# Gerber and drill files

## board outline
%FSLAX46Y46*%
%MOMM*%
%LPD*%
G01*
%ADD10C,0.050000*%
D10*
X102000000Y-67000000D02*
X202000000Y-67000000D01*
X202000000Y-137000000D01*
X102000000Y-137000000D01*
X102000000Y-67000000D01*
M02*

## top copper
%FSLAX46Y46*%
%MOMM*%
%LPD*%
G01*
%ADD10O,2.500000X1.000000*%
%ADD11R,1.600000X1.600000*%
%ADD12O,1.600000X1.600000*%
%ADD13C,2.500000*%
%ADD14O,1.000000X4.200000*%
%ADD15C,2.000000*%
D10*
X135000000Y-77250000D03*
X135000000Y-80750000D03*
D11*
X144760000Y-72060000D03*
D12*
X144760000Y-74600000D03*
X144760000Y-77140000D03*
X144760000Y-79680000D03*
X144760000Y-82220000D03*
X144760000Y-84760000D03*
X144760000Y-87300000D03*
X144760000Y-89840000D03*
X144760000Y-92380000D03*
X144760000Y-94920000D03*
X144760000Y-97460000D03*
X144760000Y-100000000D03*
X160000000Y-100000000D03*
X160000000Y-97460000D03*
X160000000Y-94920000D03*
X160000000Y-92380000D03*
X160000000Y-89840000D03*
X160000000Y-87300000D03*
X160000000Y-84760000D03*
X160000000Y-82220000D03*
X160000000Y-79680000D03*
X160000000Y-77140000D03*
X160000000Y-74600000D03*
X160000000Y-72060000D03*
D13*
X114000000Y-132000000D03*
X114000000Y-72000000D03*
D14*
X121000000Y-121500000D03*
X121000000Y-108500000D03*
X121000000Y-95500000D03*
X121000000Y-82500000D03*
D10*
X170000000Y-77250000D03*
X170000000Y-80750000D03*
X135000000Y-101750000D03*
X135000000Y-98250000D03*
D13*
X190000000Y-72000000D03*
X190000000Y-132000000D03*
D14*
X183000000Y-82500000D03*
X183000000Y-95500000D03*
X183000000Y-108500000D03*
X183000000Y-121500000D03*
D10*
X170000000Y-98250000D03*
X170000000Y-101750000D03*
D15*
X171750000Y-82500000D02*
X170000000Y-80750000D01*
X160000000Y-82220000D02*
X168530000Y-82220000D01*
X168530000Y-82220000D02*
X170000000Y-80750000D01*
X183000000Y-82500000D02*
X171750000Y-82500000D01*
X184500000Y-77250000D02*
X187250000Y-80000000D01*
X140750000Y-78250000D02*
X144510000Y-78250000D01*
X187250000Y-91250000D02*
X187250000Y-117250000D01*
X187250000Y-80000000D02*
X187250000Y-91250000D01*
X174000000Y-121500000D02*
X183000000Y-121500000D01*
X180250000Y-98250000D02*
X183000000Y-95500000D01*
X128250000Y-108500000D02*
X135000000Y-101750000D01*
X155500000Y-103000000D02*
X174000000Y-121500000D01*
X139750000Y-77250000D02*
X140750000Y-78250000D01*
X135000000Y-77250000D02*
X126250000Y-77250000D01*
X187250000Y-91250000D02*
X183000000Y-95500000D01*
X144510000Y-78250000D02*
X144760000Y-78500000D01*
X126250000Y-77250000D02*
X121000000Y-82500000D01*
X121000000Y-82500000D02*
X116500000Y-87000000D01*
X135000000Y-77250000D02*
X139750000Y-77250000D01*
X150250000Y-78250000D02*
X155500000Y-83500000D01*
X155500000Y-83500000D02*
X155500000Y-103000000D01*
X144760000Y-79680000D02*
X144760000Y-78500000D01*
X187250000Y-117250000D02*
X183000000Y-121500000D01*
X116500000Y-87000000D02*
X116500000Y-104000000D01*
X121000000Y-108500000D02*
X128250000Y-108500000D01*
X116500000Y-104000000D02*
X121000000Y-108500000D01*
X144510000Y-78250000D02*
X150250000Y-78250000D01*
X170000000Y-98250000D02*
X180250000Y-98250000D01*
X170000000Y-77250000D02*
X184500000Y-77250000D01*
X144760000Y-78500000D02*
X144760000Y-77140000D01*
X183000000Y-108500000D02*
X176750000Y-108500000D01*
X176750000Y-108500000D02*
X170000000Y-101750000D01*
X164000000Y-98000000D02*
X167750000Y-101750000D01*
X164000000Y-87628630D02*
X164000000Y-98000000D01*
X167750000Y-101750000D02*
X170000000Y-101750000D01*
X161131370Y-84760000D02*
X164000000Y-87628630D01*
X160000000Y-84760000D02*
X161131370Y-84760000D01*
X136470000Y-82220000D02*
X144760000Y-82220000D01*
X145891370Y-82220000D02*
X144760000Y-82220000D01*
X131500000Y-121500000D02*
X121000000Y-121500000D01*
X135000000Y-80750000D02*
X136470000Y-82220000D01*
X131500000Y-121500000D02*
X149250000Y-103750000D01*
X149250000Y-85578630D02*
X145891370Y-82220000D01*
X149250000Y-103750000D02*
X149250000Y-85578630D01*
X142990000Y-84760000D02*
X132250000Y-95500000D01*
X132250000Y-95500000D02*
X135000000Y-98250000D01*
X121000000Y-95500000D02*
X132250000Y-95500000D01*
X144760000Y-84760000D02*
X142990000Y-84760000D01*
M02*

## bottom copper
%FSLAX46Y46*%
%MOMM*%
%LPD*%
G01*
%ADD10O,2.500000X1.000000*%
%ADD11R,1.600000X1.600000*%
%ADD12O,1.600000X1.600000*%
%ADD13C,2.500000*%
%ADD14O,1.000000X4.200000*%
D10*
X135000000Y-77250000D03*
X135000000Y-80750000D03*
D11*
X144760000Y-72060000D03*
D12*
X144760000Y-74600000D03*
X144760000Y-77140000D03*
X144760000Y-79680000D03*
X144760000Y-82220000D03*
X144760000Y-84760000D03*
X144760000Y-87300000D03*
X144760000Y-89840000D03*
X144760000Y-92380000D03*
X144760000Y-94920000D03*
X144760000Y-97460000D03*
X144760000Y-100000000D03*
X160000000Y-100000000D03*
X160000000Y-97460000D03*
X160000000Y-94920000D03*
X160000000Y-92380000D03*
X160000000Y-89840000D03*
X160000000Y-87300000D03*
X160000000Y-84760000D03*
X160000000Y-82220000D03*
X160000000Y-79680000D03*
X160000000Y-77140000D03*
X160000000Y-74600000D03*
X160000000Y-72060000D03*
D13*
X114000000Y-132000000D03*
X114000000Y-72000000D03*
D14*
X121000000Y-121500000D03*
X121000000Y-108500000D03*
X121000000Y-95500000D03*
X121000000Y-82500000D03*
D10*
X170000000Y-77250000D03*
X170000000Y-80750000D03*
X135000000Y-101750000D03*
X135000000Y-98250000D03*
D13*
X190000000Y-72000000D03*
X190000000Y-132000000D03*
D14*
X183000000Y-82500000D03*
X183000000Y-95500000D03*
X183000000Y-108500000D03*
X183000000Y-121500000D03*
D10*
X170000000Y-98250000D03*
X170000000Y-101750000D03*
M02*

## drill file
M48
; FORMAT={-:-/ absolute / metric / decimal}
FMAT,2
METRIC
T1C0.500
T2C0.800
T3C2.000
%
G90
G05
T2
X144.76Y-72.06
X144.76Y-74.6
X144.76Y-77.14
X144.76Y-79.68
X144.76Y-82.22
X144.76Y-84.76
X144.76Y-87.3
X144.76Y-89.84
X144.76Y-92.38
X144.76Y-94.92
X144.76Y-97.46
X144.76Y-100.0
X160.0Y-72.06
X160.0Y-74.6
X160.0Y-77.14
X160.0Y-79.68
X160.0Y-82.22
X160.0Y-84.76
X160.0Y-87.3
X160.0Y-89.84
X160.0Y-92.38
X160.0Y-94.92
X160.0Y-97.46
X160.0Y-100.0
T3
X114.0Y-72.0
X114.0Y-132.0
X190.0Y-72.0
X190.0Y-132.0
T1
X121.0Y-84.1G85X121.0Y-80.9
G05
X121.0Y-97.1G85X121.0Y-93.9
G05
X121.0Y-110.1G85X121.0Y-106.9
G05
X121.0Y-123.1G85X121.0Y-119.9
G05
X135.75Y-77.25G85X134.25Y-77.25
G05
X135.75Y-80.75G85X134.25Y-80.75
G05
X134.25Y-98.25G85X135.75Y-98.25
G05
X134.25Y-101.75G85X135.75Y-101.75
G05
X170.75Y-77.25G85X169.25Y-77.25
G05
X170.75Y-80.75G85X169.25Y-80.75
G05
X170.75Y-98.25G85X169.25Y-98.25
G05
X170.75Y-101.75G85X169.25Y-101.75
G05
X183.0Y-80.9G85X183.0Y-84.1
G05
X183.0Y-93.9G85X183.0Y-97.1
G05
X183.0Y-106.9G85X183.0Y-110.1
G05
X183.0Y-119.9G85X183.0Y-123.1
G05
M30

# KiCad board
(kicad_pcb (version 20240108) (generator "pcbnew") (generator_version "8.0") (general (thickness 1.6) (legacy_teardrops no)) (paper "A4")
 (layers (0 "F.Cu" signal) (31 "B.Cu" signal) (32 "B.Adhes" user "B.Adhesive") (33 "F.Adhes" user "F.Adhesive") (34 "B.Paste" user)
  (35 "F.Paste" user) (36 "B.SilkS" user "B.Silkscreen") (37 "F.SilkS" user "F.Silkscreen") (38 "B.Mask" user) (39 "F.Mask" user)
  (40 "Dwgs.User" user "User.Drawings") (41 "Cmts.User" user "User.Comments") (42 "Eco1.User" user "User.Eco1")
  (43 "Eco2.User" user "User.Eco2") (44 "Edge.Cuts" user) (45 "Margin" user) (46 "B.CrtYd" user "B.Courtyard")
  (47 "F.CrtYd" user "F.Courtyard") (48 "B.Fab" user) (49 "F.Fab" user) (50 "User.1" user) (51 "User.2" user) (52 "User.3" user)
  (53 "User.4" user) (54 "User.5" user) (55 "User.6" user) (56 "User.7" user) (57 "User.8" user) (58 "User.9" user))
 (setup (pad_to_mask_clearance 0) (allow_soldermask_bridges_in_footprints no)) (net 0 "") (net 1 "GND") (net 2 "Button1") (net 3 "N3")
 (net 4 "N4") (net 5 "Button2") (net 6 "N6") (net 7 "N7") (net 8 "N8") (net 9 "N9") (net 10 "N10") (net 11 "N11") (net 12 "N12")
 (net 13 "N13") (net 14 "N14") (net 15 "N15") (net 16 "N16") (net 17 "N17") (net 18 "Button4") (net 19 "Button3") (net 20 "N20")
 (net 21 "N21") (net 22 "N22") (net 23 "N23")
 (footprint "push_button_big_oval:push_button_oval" (layer "F.Cu") (at 135 79 90)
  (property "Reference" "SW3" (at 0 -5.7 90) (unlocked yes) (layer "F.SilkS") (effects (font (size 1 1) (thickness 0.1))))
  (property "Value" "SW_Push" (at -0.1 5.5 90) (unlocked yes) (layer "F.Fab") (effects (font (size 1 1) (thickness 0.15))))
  (pad "1" thru_hole oval (at 1.75 0 180) (size 2.5 1) (drill oval 2 0.5) (layers "*.Cu" "*.Mask") (remove_unused_layers no) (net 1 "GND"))
  (pad "2" thru_hole oval (at -1.75 0 180) (size 2.5 1) (drill oval 2 0.5) (layers "*.Cu" "*.Mask") (remove_unused_layers no)
   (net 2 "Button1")))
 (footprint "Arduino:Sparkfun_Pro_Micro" (layer "F.Cu") (at 160 100 180)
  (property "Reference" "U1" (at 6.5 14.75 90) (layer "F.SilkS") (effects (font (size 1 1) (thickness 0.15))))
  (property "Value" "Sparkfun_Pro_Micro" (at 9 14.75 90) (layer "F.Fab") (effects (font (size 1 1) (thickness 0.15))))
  (pad "1" thru_hole rect (at 15.24 27.94 180) (size 1.6 1.6) (drill 0.8) (layers "*.Cu" "*.Mask") (remove_unused_layers no) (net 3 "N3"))
  (pad "2" thru_hole oval (at 15.24 25.4 180) (size 1.6 1.6) (drill 0.8) (layers "*.Cu" "*.Mask") (remove_unused_layers no) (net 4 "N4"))
  (pad "3" thru_hole oval (at 15.24 22.86 180) (size 1.6 1.6) (drill 0.8) (layers "*.Cu" "*.Mask") (remove_unused_layers no) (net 1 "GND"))
  (pad "4" thru_hole oval (at 15.24 20.32 180) (size 1.6 1.6) (drill 0.8) (layers "*.Cu" "*.Mask") (remove_unused_layers no) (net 1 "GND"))
  (pad "5" thru_hole oval (at 15.24 17.78 180) (size 1.6 1.6) (drill 0.8) (layers "*.Cu" "*.Mask") (remove_unused_layers no)
   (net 2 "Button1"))
  (pad "6" thru_hole oval (at 15.24 15.24 180) (size 1.6 1.6) (drill 0.8) (layers "*.Cu" "*.Mask") (remove_unused_layers no)
   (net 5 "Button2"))
  (pad "7" thru_hole oval (at 15.24 12.7 180) (size 1.6 1.6) (drill 0.8) (layers "*.Cu" "*.Mask") (remove_unused_layers no) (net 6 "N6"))
  (pad "8" thru_hole oval (at 15.24 10.16 180) (size 1.6 1.6) (drill 0.8) (layers "*.Cu" "*.Mask") (remove_unused_layers no) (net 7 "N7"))
  (pad "9" thru_hole oval (at 15.24 7.62 180) (size 1.6 1.6) (drill 0.8) (layers "*.Cu" "*.Mask") (remove_unused_layers no) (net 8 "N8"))
  (pad "10" thru_hole oval (at 15.24 5.08 180) (size 1.6 1.6) (drill 0.8) (layers "*.Cu" "*.Mask") (remove_unused_layers no) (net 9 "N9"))
  (pad "11" thru_hole oval (at 15.24 2.54 180) (size 1.6 1.6) (drill 0.8) (layers "*.Cu" "*.Mask") (remove_unused_layers no) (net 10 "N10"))
  (pad "12" thru_hole oval (at 15.24 0 180) (size 1.6 1.6) (drill 0.8) (layers "*.Cu" "*.Mask") (remove_unused_layers no) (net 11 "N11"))
  (pad "13" thru_hole oval (at 0 0 180) (size 1.6 1.6) (drill 0.8) (layers "*.Cu" "*.Mask") (remove_unused_layers no) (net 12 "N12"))
  (pad "14" thru_hole oval (at 0 2.54 180) (size 1.6 1.6) (drill 0.8) (layers "*.Cu" "*.Mask") (remove_unused_layers no) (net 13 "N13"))
  (pad "15" thru_hole oval (at 0 5.08 180) (size 1.6 1.6) (drill 0.8) (layers "*.Cu" "*.Mask") (remove_unused_layers no) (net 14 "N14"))
  (pad "16" thru_hole oval (at 0 7.62 180) (size 1.6 1.6) (drill 0.8) (layers "*.Cu" "*.Mask") (remove_unused_layers no) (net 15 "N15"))
  (pad "17" thru_hole oval (at 0 10.16 180) (size 1.6 1.6) (drill 0.8) (layers "*.Cu" "*.Mask") (remove_unused_layers no) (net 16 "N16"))
  (pad "18" thru_hole oval (at 0 12.7 180) (size 1.6 1.6) (drill 0.8) (layers "*.Cu" "*.Mask") (remove_unused_layers no) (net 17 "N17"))
  (pad "19" thru_hole oval (at 0 15.24 180) (size 1.6 1.6) (drill 0.8) (layers "*.Cu" "*.Mask") (remove_unused_layers no) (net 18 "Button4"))
  (pad "20" thru_hole oval (at 0 17.78 180) (size 1.6 1.6) (drill 0.8) (layers "*.Cu" "*.Mask") (remove_unused_layers no) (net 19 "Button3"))
  (pad "21" thru_hole oval (at 0 20.32 180) (size 1.6 1.6) (drill 0.8) (layers "*.Cu" "*.Mask") (remove_unused_layers no) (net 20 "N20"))
  (pad "22" thru_hole oval (at 0 22.86 180) (size 1.6 1.6) (drill 0.8) (layers "*.Cu" "*.Mask") (remove_unused_layers no) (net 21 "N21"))
  (pad "23" thru_hole oval (at 0 25.4 180) (size 1.6 1.6) (drill 0.8) (layers "*.Cu" "*.Mask") (remove_unused_layers no) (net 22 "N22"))
  (pad "24" thru_hole oval (at 0 27.94 180) (size 1.6 1.6) (drill 0.8) (layers "*.Cu" "*.Mask") (remove_unused_layers no) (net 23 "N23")))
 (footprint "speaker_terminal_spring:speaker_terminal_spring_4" (layer "F.Cu") (at 114 102 90)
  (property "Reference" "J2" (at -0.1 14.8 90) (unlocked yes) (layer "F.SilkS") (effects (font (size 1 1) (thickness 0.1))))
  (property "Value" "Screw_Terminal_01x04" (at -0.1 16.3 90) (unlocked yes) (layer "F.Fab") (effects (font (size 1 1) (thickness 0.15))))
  (pad "" thru_hole circle (at -30 0 180) (size 2.5 2.5) (drill 2) (layers "*.Cu" "*.Mask") (remove_unused_layers no))
  (pad "" thru_hole circle (at 30 0 180) (size 2.5 2.5) (drill 2) (layers "*.Cu" "*.Mask") (remove_unused_layers no))
  (pad "1" thru_hole oval (at -19.5 7 180) (size 1 4.2) (drill oval 0.5 3.7) (layers "*.Cu" "*.Mask") (remove_unused_layers no)
   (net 2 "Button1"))
  (pad "2" thru_hole oval (at -6.5 7 180) (size 1 4.2) (drill oval 0.5 3.7) (layers "*.Cu" "*.Mask") (remove_unused_layers no) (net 1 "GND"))
  (pad "3" thru_hole oval (at 6.5 7 180) (size 1 4.2) (drill oval 0.5 3.7) (layers "*.Cu" "*.Mask") (remove_unused_layers no)
   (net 5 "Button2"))
  (pad "4" thru_hole oval (at 19.5 7 180) (size 1 4.2) (drill oval 0.5 3.7) (layers "*.Cu" "*.Mask") (remove_unused_layers no) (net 1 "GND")))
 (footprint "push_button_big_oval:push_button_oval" (layer "F.Cu") (at 170 79 90)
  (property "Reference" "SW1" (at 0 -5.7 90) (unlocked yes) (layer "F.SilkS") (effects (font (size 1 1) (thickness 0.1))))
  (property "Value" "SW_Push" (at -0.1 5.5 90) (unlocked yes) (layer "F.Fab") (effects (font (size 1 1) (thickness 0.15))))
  (pad "1" thru_hole oval (at 1.75 0 180) (size 2.5 1) (drill oval 2 0.5) (layers "*.Cu" "*.Mask") (remove_unused_layers no) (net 1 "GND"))
  (pad "2" thru_hole oval (at -1.75 0 180) (size 2.5 1) (drill oval 2 0.5) (layers "*.Cu" "*.Mask") (remove_unused_layers no)
   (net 19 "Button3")))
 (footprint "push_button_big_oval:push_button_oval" (layer "F.Cu") (at 135 100 -90)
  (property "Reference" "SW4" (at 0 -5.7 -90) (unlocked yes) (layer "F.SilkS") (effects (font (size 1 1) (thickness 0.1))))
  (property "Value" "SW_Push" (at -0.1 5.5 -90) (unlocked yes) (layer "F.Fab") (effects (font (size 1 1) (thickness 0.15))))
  (pad "1" thru_hole oval (at 1.75 0) (size 2.5 1) (drill oval 2 0.5) (layers "*.Cu" "*.Mask") (remove_unused_layers no) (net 1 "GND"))
  (pad "2" thru_hole oval (at -1.75 0) (size 2.5 1) (drill oval 2 0.5) (layers "*.Cu" "*.Mask") (remove_unused_layers no) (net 5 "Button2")))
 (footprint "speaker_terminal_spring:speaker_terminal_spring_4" (layer "F.Cu") (at 190 102 -90)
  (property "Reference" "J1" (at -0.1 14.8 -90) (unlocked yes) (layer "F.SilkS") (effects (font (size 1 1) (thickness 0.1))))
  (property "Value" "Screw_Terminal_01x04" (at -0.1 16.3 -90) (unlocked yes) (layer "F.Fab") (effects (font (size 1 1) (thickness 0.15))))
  (pad "" thru_hole circle (at -30 0) (size 2.5 2.5) (drill 2) (layers "*.Cu" "*.Mask") (remove_unused_layers no))
  (pad "" thru_hole circle (at 30 0) (size 2.5 2.5) (drill 2) (layers "*.Cu" "*.Mask") (remove_unused_layers no))
  (pad "1" thru_hole oval (at -19.5 7) (size 1 4.2) (drill oval 0.5 3.7) (layers "*.Cu" "*.Mask") (remove_unused_layers no)
   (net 19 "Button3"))
  (pad "2" thru_hole oval (at -6.5 7) (size 1 4.2) (drill oval 0.5 3.7) (layers "*.Cu" "*.Mask") (remove_unused_layers no) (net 1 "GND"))
  (pad "3" thru_hole oval (at 6.5 7) (size 1 4.2) (drill oval 0.5 3.7) (layers "*.Cu" "*.Mask") (remove_unused_layers no) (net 18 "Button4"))
  (pad "4" thru_hole oval (at 19.5 7) (size 1 4.2) (drill oval 0.5 3.7) (layers "*.Cu" "*.Mask") (remove_unused_layers no) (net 1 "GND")))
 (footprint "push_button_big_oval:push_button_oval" (layer "F.Cu") (at 170 100 90)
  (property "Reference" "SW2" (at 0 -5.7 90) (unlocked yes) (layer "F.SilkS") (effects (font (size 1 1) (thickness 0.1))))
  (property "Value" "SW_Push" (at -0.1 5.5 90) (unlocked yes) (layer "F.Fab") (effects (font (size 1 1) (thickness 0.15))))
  (pad "1" thru_hole oval (at 1.75 0 180) (size 2.5 1) (drill oval 2 0.5) (layers "*.Cu" "*.Mask") (remove_unused_layers no) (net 1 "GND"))
  (pad "2" thru_hole oval (at -1.75 0 180) (size 2.5 1) (drill oval 2 0.5) (layers "*.Cu" "*.Mask") (remove_unused_layers no)
   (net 18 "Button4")))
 (gr_rect (start 102 67) (end 202 137) (stroke (width 0.05) (type default)) (fill none) (layer "Edge.Cuts"))
 (segment (start 171.75 82.5) (end 170 80.75) (width 2) (layer "F.Cu") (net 19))
 (segment (start 160 82.22) (end 168.53 82.22) (width 2) (layer "F.Cu") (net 19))
 (segment (start 168.53 82.22) (end 170 80.75) (width 2) (layer "F.Cu") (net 19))
 (segment (start 183 82.5) (end 171.75 82.5) (width 2) (layer "F.Cu") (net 19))
 (segment (start 184.5 77.25) (end 187.25 80) (width 2) (layer "F.Cu") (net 1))
 (segment (start 140.75 78.25) (end 144.51 78.25) (width 2) (layer "F.Cu") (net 1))
 (segment (start 187.25 91.25) (end 187.25 117.25) (width 2) (layer "F.Cu") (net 1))
 (segment (start 187.25 80) (end 187.25 91.25) (width 2) (layer "F.Cu") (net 1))
 (segment (start 174 121.5) (end 183 121.5) (width 2) (layer "F.Cu") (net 1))
 (segment (start 180.25 98.25) (end 183 95.5) (width 2) (layer "F.Cu") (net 1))
 (segment (start 128.25 108.5) (end 135 101.75) (width 2) (layer "F.Cu") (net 1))
 (segment (start 155.5 103) (end 174 121.5) (width 2) (layer "F.Cu") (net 1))
 (segment (start 139.75 77.25) (end 140.75 78.25) (width 2) (layer "F.Cu") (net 1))
 (segment (start 135 77.25) (end 126.25 77.25) (width 2) (layer "F.Cu") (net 1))
 (segment (start 187.25 91.25) (end 183 95.5) (width 2) (layer "F.Cu") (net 1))
 (segment (start 144.51 78.25) (end 144.76 78.5) (width 2) (layer "F.Cu") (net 1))
 (segment (start 126.25 77.25) (end 121 82.5) (width 2) (layer "F.Cu") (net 1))
 (segment (start 121 82.5) (end 116.5 87) (width 2) (layer "F.Cu") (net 1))
 (segment (start 135 77.25) (end 139.75 77.25) (width 2) (layer "F.Cu") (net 1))
 (segment (start 150.25 78.25) (end 155.5 83.5) (width 2) (layer "F.Cu") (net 1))
 (segment (start 155.5 83.5) (end 155.5 103) (width 2) (layer "F.Cu") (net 1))
 (segment (start 144.76 79.68) (end 144.76 78.5) (width 2) (layer "F.Cu") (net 1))
 (segment (start 187.25 117.25) (end 183 121.5) (width 2) (layer "F.Cu") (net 1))
 (segment (start 116.5 87) (end 116.5 104) (width 2) (layer "F.Cu") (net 1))
 (segment (start 121 108.5) (end 128.25 108.5) (width 2) (layer "F.Cu") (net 1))
 (segment (start 116.5 104) (end 121 108.5) (width 2) (layer "F.Cu") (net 1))
 (segment (start 144.51 78.25) (end 150.25 78.25) (width 2) (layer "F.Cu") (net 1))
 (segment (start 170 98.25) (end 180.25 98.25) (width 2) (layer "F.Cu") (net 1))
 (segment (start 170 77.25) (end 184.5 77.25) (width 2) (layer "F.Cu") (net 1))
 (segment (start 144.76 78.5) (end 144.76 77.14) (width 2) (layer "F.Cu") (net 1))
 (segment (start 183 108.5) (end 176.75 108.5) (width 2) (layer "F.Cu") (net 18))
 (segment (start 176.75 108.5) (end 170 101.75) (width 2) (layer "F.Cu") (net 18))
 (segment (start 164 98) (end 167.75 101.75) (width 2) (layer "F.Cu") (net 18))
 (segment (start 164 87.62863) (end 164 98) (width 2) (layer "F.Cu") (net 18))
 (segment (start 167.75 101.75) (end 170 101.75) (width 2) (layer "F.Cu") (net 18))
 (segment (start 161.13137 84.76) (end 164 87.62863) (width 2) (layer "F.Cu") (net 18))
 (segment (start 160 84.76) (end 161.13137 84.76) (width 2) (layer "F.Cu") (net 18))
 (segment (start 136.47 82.22) (end 144.76 82.22) (width 2) (layer "F.Cu") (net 2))
 (segment (start 145.89137 82.22) (end 144.76 82.22) (width 2) (layer "F.Cu") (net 2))
 (segment (start 131.5 121.5) (end 121 121.5) (width 2) (layer "F.Cu") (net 2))
 (segment (start 135 80.75) (end 136.47 82.22) (width 2) (layer "F.Cu") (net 2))
 (segment (start 131.5 121.5) (end 149.25 103.75) (width 2) (layer "F.Cu") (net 2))
 (segment (start 149.25 85.57863) (end 145.89137 82.22) (width 2) (layer "F.Cu") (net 2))
 (segment (start 149.25 103.75) (end 149.25 85.57863) (width 2) (layer "F.Cu") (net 2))
 (segment (start 142.99 84.76) (end 132.25 95.5) (width 2) (layer "F.Cu") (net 5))
 (segment (start 132.25 95.5) (end 135 98.25) (width 2) (layer "F.Cu") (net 5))
 (segment (start 121 95.5) (end 132.25 95.5) (width 2) (layer "F.Cu") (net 5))
 (segment (start 144.76 84.76) (end 142.99 84.76) (width 2) (layer "F.Cu") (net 5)))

